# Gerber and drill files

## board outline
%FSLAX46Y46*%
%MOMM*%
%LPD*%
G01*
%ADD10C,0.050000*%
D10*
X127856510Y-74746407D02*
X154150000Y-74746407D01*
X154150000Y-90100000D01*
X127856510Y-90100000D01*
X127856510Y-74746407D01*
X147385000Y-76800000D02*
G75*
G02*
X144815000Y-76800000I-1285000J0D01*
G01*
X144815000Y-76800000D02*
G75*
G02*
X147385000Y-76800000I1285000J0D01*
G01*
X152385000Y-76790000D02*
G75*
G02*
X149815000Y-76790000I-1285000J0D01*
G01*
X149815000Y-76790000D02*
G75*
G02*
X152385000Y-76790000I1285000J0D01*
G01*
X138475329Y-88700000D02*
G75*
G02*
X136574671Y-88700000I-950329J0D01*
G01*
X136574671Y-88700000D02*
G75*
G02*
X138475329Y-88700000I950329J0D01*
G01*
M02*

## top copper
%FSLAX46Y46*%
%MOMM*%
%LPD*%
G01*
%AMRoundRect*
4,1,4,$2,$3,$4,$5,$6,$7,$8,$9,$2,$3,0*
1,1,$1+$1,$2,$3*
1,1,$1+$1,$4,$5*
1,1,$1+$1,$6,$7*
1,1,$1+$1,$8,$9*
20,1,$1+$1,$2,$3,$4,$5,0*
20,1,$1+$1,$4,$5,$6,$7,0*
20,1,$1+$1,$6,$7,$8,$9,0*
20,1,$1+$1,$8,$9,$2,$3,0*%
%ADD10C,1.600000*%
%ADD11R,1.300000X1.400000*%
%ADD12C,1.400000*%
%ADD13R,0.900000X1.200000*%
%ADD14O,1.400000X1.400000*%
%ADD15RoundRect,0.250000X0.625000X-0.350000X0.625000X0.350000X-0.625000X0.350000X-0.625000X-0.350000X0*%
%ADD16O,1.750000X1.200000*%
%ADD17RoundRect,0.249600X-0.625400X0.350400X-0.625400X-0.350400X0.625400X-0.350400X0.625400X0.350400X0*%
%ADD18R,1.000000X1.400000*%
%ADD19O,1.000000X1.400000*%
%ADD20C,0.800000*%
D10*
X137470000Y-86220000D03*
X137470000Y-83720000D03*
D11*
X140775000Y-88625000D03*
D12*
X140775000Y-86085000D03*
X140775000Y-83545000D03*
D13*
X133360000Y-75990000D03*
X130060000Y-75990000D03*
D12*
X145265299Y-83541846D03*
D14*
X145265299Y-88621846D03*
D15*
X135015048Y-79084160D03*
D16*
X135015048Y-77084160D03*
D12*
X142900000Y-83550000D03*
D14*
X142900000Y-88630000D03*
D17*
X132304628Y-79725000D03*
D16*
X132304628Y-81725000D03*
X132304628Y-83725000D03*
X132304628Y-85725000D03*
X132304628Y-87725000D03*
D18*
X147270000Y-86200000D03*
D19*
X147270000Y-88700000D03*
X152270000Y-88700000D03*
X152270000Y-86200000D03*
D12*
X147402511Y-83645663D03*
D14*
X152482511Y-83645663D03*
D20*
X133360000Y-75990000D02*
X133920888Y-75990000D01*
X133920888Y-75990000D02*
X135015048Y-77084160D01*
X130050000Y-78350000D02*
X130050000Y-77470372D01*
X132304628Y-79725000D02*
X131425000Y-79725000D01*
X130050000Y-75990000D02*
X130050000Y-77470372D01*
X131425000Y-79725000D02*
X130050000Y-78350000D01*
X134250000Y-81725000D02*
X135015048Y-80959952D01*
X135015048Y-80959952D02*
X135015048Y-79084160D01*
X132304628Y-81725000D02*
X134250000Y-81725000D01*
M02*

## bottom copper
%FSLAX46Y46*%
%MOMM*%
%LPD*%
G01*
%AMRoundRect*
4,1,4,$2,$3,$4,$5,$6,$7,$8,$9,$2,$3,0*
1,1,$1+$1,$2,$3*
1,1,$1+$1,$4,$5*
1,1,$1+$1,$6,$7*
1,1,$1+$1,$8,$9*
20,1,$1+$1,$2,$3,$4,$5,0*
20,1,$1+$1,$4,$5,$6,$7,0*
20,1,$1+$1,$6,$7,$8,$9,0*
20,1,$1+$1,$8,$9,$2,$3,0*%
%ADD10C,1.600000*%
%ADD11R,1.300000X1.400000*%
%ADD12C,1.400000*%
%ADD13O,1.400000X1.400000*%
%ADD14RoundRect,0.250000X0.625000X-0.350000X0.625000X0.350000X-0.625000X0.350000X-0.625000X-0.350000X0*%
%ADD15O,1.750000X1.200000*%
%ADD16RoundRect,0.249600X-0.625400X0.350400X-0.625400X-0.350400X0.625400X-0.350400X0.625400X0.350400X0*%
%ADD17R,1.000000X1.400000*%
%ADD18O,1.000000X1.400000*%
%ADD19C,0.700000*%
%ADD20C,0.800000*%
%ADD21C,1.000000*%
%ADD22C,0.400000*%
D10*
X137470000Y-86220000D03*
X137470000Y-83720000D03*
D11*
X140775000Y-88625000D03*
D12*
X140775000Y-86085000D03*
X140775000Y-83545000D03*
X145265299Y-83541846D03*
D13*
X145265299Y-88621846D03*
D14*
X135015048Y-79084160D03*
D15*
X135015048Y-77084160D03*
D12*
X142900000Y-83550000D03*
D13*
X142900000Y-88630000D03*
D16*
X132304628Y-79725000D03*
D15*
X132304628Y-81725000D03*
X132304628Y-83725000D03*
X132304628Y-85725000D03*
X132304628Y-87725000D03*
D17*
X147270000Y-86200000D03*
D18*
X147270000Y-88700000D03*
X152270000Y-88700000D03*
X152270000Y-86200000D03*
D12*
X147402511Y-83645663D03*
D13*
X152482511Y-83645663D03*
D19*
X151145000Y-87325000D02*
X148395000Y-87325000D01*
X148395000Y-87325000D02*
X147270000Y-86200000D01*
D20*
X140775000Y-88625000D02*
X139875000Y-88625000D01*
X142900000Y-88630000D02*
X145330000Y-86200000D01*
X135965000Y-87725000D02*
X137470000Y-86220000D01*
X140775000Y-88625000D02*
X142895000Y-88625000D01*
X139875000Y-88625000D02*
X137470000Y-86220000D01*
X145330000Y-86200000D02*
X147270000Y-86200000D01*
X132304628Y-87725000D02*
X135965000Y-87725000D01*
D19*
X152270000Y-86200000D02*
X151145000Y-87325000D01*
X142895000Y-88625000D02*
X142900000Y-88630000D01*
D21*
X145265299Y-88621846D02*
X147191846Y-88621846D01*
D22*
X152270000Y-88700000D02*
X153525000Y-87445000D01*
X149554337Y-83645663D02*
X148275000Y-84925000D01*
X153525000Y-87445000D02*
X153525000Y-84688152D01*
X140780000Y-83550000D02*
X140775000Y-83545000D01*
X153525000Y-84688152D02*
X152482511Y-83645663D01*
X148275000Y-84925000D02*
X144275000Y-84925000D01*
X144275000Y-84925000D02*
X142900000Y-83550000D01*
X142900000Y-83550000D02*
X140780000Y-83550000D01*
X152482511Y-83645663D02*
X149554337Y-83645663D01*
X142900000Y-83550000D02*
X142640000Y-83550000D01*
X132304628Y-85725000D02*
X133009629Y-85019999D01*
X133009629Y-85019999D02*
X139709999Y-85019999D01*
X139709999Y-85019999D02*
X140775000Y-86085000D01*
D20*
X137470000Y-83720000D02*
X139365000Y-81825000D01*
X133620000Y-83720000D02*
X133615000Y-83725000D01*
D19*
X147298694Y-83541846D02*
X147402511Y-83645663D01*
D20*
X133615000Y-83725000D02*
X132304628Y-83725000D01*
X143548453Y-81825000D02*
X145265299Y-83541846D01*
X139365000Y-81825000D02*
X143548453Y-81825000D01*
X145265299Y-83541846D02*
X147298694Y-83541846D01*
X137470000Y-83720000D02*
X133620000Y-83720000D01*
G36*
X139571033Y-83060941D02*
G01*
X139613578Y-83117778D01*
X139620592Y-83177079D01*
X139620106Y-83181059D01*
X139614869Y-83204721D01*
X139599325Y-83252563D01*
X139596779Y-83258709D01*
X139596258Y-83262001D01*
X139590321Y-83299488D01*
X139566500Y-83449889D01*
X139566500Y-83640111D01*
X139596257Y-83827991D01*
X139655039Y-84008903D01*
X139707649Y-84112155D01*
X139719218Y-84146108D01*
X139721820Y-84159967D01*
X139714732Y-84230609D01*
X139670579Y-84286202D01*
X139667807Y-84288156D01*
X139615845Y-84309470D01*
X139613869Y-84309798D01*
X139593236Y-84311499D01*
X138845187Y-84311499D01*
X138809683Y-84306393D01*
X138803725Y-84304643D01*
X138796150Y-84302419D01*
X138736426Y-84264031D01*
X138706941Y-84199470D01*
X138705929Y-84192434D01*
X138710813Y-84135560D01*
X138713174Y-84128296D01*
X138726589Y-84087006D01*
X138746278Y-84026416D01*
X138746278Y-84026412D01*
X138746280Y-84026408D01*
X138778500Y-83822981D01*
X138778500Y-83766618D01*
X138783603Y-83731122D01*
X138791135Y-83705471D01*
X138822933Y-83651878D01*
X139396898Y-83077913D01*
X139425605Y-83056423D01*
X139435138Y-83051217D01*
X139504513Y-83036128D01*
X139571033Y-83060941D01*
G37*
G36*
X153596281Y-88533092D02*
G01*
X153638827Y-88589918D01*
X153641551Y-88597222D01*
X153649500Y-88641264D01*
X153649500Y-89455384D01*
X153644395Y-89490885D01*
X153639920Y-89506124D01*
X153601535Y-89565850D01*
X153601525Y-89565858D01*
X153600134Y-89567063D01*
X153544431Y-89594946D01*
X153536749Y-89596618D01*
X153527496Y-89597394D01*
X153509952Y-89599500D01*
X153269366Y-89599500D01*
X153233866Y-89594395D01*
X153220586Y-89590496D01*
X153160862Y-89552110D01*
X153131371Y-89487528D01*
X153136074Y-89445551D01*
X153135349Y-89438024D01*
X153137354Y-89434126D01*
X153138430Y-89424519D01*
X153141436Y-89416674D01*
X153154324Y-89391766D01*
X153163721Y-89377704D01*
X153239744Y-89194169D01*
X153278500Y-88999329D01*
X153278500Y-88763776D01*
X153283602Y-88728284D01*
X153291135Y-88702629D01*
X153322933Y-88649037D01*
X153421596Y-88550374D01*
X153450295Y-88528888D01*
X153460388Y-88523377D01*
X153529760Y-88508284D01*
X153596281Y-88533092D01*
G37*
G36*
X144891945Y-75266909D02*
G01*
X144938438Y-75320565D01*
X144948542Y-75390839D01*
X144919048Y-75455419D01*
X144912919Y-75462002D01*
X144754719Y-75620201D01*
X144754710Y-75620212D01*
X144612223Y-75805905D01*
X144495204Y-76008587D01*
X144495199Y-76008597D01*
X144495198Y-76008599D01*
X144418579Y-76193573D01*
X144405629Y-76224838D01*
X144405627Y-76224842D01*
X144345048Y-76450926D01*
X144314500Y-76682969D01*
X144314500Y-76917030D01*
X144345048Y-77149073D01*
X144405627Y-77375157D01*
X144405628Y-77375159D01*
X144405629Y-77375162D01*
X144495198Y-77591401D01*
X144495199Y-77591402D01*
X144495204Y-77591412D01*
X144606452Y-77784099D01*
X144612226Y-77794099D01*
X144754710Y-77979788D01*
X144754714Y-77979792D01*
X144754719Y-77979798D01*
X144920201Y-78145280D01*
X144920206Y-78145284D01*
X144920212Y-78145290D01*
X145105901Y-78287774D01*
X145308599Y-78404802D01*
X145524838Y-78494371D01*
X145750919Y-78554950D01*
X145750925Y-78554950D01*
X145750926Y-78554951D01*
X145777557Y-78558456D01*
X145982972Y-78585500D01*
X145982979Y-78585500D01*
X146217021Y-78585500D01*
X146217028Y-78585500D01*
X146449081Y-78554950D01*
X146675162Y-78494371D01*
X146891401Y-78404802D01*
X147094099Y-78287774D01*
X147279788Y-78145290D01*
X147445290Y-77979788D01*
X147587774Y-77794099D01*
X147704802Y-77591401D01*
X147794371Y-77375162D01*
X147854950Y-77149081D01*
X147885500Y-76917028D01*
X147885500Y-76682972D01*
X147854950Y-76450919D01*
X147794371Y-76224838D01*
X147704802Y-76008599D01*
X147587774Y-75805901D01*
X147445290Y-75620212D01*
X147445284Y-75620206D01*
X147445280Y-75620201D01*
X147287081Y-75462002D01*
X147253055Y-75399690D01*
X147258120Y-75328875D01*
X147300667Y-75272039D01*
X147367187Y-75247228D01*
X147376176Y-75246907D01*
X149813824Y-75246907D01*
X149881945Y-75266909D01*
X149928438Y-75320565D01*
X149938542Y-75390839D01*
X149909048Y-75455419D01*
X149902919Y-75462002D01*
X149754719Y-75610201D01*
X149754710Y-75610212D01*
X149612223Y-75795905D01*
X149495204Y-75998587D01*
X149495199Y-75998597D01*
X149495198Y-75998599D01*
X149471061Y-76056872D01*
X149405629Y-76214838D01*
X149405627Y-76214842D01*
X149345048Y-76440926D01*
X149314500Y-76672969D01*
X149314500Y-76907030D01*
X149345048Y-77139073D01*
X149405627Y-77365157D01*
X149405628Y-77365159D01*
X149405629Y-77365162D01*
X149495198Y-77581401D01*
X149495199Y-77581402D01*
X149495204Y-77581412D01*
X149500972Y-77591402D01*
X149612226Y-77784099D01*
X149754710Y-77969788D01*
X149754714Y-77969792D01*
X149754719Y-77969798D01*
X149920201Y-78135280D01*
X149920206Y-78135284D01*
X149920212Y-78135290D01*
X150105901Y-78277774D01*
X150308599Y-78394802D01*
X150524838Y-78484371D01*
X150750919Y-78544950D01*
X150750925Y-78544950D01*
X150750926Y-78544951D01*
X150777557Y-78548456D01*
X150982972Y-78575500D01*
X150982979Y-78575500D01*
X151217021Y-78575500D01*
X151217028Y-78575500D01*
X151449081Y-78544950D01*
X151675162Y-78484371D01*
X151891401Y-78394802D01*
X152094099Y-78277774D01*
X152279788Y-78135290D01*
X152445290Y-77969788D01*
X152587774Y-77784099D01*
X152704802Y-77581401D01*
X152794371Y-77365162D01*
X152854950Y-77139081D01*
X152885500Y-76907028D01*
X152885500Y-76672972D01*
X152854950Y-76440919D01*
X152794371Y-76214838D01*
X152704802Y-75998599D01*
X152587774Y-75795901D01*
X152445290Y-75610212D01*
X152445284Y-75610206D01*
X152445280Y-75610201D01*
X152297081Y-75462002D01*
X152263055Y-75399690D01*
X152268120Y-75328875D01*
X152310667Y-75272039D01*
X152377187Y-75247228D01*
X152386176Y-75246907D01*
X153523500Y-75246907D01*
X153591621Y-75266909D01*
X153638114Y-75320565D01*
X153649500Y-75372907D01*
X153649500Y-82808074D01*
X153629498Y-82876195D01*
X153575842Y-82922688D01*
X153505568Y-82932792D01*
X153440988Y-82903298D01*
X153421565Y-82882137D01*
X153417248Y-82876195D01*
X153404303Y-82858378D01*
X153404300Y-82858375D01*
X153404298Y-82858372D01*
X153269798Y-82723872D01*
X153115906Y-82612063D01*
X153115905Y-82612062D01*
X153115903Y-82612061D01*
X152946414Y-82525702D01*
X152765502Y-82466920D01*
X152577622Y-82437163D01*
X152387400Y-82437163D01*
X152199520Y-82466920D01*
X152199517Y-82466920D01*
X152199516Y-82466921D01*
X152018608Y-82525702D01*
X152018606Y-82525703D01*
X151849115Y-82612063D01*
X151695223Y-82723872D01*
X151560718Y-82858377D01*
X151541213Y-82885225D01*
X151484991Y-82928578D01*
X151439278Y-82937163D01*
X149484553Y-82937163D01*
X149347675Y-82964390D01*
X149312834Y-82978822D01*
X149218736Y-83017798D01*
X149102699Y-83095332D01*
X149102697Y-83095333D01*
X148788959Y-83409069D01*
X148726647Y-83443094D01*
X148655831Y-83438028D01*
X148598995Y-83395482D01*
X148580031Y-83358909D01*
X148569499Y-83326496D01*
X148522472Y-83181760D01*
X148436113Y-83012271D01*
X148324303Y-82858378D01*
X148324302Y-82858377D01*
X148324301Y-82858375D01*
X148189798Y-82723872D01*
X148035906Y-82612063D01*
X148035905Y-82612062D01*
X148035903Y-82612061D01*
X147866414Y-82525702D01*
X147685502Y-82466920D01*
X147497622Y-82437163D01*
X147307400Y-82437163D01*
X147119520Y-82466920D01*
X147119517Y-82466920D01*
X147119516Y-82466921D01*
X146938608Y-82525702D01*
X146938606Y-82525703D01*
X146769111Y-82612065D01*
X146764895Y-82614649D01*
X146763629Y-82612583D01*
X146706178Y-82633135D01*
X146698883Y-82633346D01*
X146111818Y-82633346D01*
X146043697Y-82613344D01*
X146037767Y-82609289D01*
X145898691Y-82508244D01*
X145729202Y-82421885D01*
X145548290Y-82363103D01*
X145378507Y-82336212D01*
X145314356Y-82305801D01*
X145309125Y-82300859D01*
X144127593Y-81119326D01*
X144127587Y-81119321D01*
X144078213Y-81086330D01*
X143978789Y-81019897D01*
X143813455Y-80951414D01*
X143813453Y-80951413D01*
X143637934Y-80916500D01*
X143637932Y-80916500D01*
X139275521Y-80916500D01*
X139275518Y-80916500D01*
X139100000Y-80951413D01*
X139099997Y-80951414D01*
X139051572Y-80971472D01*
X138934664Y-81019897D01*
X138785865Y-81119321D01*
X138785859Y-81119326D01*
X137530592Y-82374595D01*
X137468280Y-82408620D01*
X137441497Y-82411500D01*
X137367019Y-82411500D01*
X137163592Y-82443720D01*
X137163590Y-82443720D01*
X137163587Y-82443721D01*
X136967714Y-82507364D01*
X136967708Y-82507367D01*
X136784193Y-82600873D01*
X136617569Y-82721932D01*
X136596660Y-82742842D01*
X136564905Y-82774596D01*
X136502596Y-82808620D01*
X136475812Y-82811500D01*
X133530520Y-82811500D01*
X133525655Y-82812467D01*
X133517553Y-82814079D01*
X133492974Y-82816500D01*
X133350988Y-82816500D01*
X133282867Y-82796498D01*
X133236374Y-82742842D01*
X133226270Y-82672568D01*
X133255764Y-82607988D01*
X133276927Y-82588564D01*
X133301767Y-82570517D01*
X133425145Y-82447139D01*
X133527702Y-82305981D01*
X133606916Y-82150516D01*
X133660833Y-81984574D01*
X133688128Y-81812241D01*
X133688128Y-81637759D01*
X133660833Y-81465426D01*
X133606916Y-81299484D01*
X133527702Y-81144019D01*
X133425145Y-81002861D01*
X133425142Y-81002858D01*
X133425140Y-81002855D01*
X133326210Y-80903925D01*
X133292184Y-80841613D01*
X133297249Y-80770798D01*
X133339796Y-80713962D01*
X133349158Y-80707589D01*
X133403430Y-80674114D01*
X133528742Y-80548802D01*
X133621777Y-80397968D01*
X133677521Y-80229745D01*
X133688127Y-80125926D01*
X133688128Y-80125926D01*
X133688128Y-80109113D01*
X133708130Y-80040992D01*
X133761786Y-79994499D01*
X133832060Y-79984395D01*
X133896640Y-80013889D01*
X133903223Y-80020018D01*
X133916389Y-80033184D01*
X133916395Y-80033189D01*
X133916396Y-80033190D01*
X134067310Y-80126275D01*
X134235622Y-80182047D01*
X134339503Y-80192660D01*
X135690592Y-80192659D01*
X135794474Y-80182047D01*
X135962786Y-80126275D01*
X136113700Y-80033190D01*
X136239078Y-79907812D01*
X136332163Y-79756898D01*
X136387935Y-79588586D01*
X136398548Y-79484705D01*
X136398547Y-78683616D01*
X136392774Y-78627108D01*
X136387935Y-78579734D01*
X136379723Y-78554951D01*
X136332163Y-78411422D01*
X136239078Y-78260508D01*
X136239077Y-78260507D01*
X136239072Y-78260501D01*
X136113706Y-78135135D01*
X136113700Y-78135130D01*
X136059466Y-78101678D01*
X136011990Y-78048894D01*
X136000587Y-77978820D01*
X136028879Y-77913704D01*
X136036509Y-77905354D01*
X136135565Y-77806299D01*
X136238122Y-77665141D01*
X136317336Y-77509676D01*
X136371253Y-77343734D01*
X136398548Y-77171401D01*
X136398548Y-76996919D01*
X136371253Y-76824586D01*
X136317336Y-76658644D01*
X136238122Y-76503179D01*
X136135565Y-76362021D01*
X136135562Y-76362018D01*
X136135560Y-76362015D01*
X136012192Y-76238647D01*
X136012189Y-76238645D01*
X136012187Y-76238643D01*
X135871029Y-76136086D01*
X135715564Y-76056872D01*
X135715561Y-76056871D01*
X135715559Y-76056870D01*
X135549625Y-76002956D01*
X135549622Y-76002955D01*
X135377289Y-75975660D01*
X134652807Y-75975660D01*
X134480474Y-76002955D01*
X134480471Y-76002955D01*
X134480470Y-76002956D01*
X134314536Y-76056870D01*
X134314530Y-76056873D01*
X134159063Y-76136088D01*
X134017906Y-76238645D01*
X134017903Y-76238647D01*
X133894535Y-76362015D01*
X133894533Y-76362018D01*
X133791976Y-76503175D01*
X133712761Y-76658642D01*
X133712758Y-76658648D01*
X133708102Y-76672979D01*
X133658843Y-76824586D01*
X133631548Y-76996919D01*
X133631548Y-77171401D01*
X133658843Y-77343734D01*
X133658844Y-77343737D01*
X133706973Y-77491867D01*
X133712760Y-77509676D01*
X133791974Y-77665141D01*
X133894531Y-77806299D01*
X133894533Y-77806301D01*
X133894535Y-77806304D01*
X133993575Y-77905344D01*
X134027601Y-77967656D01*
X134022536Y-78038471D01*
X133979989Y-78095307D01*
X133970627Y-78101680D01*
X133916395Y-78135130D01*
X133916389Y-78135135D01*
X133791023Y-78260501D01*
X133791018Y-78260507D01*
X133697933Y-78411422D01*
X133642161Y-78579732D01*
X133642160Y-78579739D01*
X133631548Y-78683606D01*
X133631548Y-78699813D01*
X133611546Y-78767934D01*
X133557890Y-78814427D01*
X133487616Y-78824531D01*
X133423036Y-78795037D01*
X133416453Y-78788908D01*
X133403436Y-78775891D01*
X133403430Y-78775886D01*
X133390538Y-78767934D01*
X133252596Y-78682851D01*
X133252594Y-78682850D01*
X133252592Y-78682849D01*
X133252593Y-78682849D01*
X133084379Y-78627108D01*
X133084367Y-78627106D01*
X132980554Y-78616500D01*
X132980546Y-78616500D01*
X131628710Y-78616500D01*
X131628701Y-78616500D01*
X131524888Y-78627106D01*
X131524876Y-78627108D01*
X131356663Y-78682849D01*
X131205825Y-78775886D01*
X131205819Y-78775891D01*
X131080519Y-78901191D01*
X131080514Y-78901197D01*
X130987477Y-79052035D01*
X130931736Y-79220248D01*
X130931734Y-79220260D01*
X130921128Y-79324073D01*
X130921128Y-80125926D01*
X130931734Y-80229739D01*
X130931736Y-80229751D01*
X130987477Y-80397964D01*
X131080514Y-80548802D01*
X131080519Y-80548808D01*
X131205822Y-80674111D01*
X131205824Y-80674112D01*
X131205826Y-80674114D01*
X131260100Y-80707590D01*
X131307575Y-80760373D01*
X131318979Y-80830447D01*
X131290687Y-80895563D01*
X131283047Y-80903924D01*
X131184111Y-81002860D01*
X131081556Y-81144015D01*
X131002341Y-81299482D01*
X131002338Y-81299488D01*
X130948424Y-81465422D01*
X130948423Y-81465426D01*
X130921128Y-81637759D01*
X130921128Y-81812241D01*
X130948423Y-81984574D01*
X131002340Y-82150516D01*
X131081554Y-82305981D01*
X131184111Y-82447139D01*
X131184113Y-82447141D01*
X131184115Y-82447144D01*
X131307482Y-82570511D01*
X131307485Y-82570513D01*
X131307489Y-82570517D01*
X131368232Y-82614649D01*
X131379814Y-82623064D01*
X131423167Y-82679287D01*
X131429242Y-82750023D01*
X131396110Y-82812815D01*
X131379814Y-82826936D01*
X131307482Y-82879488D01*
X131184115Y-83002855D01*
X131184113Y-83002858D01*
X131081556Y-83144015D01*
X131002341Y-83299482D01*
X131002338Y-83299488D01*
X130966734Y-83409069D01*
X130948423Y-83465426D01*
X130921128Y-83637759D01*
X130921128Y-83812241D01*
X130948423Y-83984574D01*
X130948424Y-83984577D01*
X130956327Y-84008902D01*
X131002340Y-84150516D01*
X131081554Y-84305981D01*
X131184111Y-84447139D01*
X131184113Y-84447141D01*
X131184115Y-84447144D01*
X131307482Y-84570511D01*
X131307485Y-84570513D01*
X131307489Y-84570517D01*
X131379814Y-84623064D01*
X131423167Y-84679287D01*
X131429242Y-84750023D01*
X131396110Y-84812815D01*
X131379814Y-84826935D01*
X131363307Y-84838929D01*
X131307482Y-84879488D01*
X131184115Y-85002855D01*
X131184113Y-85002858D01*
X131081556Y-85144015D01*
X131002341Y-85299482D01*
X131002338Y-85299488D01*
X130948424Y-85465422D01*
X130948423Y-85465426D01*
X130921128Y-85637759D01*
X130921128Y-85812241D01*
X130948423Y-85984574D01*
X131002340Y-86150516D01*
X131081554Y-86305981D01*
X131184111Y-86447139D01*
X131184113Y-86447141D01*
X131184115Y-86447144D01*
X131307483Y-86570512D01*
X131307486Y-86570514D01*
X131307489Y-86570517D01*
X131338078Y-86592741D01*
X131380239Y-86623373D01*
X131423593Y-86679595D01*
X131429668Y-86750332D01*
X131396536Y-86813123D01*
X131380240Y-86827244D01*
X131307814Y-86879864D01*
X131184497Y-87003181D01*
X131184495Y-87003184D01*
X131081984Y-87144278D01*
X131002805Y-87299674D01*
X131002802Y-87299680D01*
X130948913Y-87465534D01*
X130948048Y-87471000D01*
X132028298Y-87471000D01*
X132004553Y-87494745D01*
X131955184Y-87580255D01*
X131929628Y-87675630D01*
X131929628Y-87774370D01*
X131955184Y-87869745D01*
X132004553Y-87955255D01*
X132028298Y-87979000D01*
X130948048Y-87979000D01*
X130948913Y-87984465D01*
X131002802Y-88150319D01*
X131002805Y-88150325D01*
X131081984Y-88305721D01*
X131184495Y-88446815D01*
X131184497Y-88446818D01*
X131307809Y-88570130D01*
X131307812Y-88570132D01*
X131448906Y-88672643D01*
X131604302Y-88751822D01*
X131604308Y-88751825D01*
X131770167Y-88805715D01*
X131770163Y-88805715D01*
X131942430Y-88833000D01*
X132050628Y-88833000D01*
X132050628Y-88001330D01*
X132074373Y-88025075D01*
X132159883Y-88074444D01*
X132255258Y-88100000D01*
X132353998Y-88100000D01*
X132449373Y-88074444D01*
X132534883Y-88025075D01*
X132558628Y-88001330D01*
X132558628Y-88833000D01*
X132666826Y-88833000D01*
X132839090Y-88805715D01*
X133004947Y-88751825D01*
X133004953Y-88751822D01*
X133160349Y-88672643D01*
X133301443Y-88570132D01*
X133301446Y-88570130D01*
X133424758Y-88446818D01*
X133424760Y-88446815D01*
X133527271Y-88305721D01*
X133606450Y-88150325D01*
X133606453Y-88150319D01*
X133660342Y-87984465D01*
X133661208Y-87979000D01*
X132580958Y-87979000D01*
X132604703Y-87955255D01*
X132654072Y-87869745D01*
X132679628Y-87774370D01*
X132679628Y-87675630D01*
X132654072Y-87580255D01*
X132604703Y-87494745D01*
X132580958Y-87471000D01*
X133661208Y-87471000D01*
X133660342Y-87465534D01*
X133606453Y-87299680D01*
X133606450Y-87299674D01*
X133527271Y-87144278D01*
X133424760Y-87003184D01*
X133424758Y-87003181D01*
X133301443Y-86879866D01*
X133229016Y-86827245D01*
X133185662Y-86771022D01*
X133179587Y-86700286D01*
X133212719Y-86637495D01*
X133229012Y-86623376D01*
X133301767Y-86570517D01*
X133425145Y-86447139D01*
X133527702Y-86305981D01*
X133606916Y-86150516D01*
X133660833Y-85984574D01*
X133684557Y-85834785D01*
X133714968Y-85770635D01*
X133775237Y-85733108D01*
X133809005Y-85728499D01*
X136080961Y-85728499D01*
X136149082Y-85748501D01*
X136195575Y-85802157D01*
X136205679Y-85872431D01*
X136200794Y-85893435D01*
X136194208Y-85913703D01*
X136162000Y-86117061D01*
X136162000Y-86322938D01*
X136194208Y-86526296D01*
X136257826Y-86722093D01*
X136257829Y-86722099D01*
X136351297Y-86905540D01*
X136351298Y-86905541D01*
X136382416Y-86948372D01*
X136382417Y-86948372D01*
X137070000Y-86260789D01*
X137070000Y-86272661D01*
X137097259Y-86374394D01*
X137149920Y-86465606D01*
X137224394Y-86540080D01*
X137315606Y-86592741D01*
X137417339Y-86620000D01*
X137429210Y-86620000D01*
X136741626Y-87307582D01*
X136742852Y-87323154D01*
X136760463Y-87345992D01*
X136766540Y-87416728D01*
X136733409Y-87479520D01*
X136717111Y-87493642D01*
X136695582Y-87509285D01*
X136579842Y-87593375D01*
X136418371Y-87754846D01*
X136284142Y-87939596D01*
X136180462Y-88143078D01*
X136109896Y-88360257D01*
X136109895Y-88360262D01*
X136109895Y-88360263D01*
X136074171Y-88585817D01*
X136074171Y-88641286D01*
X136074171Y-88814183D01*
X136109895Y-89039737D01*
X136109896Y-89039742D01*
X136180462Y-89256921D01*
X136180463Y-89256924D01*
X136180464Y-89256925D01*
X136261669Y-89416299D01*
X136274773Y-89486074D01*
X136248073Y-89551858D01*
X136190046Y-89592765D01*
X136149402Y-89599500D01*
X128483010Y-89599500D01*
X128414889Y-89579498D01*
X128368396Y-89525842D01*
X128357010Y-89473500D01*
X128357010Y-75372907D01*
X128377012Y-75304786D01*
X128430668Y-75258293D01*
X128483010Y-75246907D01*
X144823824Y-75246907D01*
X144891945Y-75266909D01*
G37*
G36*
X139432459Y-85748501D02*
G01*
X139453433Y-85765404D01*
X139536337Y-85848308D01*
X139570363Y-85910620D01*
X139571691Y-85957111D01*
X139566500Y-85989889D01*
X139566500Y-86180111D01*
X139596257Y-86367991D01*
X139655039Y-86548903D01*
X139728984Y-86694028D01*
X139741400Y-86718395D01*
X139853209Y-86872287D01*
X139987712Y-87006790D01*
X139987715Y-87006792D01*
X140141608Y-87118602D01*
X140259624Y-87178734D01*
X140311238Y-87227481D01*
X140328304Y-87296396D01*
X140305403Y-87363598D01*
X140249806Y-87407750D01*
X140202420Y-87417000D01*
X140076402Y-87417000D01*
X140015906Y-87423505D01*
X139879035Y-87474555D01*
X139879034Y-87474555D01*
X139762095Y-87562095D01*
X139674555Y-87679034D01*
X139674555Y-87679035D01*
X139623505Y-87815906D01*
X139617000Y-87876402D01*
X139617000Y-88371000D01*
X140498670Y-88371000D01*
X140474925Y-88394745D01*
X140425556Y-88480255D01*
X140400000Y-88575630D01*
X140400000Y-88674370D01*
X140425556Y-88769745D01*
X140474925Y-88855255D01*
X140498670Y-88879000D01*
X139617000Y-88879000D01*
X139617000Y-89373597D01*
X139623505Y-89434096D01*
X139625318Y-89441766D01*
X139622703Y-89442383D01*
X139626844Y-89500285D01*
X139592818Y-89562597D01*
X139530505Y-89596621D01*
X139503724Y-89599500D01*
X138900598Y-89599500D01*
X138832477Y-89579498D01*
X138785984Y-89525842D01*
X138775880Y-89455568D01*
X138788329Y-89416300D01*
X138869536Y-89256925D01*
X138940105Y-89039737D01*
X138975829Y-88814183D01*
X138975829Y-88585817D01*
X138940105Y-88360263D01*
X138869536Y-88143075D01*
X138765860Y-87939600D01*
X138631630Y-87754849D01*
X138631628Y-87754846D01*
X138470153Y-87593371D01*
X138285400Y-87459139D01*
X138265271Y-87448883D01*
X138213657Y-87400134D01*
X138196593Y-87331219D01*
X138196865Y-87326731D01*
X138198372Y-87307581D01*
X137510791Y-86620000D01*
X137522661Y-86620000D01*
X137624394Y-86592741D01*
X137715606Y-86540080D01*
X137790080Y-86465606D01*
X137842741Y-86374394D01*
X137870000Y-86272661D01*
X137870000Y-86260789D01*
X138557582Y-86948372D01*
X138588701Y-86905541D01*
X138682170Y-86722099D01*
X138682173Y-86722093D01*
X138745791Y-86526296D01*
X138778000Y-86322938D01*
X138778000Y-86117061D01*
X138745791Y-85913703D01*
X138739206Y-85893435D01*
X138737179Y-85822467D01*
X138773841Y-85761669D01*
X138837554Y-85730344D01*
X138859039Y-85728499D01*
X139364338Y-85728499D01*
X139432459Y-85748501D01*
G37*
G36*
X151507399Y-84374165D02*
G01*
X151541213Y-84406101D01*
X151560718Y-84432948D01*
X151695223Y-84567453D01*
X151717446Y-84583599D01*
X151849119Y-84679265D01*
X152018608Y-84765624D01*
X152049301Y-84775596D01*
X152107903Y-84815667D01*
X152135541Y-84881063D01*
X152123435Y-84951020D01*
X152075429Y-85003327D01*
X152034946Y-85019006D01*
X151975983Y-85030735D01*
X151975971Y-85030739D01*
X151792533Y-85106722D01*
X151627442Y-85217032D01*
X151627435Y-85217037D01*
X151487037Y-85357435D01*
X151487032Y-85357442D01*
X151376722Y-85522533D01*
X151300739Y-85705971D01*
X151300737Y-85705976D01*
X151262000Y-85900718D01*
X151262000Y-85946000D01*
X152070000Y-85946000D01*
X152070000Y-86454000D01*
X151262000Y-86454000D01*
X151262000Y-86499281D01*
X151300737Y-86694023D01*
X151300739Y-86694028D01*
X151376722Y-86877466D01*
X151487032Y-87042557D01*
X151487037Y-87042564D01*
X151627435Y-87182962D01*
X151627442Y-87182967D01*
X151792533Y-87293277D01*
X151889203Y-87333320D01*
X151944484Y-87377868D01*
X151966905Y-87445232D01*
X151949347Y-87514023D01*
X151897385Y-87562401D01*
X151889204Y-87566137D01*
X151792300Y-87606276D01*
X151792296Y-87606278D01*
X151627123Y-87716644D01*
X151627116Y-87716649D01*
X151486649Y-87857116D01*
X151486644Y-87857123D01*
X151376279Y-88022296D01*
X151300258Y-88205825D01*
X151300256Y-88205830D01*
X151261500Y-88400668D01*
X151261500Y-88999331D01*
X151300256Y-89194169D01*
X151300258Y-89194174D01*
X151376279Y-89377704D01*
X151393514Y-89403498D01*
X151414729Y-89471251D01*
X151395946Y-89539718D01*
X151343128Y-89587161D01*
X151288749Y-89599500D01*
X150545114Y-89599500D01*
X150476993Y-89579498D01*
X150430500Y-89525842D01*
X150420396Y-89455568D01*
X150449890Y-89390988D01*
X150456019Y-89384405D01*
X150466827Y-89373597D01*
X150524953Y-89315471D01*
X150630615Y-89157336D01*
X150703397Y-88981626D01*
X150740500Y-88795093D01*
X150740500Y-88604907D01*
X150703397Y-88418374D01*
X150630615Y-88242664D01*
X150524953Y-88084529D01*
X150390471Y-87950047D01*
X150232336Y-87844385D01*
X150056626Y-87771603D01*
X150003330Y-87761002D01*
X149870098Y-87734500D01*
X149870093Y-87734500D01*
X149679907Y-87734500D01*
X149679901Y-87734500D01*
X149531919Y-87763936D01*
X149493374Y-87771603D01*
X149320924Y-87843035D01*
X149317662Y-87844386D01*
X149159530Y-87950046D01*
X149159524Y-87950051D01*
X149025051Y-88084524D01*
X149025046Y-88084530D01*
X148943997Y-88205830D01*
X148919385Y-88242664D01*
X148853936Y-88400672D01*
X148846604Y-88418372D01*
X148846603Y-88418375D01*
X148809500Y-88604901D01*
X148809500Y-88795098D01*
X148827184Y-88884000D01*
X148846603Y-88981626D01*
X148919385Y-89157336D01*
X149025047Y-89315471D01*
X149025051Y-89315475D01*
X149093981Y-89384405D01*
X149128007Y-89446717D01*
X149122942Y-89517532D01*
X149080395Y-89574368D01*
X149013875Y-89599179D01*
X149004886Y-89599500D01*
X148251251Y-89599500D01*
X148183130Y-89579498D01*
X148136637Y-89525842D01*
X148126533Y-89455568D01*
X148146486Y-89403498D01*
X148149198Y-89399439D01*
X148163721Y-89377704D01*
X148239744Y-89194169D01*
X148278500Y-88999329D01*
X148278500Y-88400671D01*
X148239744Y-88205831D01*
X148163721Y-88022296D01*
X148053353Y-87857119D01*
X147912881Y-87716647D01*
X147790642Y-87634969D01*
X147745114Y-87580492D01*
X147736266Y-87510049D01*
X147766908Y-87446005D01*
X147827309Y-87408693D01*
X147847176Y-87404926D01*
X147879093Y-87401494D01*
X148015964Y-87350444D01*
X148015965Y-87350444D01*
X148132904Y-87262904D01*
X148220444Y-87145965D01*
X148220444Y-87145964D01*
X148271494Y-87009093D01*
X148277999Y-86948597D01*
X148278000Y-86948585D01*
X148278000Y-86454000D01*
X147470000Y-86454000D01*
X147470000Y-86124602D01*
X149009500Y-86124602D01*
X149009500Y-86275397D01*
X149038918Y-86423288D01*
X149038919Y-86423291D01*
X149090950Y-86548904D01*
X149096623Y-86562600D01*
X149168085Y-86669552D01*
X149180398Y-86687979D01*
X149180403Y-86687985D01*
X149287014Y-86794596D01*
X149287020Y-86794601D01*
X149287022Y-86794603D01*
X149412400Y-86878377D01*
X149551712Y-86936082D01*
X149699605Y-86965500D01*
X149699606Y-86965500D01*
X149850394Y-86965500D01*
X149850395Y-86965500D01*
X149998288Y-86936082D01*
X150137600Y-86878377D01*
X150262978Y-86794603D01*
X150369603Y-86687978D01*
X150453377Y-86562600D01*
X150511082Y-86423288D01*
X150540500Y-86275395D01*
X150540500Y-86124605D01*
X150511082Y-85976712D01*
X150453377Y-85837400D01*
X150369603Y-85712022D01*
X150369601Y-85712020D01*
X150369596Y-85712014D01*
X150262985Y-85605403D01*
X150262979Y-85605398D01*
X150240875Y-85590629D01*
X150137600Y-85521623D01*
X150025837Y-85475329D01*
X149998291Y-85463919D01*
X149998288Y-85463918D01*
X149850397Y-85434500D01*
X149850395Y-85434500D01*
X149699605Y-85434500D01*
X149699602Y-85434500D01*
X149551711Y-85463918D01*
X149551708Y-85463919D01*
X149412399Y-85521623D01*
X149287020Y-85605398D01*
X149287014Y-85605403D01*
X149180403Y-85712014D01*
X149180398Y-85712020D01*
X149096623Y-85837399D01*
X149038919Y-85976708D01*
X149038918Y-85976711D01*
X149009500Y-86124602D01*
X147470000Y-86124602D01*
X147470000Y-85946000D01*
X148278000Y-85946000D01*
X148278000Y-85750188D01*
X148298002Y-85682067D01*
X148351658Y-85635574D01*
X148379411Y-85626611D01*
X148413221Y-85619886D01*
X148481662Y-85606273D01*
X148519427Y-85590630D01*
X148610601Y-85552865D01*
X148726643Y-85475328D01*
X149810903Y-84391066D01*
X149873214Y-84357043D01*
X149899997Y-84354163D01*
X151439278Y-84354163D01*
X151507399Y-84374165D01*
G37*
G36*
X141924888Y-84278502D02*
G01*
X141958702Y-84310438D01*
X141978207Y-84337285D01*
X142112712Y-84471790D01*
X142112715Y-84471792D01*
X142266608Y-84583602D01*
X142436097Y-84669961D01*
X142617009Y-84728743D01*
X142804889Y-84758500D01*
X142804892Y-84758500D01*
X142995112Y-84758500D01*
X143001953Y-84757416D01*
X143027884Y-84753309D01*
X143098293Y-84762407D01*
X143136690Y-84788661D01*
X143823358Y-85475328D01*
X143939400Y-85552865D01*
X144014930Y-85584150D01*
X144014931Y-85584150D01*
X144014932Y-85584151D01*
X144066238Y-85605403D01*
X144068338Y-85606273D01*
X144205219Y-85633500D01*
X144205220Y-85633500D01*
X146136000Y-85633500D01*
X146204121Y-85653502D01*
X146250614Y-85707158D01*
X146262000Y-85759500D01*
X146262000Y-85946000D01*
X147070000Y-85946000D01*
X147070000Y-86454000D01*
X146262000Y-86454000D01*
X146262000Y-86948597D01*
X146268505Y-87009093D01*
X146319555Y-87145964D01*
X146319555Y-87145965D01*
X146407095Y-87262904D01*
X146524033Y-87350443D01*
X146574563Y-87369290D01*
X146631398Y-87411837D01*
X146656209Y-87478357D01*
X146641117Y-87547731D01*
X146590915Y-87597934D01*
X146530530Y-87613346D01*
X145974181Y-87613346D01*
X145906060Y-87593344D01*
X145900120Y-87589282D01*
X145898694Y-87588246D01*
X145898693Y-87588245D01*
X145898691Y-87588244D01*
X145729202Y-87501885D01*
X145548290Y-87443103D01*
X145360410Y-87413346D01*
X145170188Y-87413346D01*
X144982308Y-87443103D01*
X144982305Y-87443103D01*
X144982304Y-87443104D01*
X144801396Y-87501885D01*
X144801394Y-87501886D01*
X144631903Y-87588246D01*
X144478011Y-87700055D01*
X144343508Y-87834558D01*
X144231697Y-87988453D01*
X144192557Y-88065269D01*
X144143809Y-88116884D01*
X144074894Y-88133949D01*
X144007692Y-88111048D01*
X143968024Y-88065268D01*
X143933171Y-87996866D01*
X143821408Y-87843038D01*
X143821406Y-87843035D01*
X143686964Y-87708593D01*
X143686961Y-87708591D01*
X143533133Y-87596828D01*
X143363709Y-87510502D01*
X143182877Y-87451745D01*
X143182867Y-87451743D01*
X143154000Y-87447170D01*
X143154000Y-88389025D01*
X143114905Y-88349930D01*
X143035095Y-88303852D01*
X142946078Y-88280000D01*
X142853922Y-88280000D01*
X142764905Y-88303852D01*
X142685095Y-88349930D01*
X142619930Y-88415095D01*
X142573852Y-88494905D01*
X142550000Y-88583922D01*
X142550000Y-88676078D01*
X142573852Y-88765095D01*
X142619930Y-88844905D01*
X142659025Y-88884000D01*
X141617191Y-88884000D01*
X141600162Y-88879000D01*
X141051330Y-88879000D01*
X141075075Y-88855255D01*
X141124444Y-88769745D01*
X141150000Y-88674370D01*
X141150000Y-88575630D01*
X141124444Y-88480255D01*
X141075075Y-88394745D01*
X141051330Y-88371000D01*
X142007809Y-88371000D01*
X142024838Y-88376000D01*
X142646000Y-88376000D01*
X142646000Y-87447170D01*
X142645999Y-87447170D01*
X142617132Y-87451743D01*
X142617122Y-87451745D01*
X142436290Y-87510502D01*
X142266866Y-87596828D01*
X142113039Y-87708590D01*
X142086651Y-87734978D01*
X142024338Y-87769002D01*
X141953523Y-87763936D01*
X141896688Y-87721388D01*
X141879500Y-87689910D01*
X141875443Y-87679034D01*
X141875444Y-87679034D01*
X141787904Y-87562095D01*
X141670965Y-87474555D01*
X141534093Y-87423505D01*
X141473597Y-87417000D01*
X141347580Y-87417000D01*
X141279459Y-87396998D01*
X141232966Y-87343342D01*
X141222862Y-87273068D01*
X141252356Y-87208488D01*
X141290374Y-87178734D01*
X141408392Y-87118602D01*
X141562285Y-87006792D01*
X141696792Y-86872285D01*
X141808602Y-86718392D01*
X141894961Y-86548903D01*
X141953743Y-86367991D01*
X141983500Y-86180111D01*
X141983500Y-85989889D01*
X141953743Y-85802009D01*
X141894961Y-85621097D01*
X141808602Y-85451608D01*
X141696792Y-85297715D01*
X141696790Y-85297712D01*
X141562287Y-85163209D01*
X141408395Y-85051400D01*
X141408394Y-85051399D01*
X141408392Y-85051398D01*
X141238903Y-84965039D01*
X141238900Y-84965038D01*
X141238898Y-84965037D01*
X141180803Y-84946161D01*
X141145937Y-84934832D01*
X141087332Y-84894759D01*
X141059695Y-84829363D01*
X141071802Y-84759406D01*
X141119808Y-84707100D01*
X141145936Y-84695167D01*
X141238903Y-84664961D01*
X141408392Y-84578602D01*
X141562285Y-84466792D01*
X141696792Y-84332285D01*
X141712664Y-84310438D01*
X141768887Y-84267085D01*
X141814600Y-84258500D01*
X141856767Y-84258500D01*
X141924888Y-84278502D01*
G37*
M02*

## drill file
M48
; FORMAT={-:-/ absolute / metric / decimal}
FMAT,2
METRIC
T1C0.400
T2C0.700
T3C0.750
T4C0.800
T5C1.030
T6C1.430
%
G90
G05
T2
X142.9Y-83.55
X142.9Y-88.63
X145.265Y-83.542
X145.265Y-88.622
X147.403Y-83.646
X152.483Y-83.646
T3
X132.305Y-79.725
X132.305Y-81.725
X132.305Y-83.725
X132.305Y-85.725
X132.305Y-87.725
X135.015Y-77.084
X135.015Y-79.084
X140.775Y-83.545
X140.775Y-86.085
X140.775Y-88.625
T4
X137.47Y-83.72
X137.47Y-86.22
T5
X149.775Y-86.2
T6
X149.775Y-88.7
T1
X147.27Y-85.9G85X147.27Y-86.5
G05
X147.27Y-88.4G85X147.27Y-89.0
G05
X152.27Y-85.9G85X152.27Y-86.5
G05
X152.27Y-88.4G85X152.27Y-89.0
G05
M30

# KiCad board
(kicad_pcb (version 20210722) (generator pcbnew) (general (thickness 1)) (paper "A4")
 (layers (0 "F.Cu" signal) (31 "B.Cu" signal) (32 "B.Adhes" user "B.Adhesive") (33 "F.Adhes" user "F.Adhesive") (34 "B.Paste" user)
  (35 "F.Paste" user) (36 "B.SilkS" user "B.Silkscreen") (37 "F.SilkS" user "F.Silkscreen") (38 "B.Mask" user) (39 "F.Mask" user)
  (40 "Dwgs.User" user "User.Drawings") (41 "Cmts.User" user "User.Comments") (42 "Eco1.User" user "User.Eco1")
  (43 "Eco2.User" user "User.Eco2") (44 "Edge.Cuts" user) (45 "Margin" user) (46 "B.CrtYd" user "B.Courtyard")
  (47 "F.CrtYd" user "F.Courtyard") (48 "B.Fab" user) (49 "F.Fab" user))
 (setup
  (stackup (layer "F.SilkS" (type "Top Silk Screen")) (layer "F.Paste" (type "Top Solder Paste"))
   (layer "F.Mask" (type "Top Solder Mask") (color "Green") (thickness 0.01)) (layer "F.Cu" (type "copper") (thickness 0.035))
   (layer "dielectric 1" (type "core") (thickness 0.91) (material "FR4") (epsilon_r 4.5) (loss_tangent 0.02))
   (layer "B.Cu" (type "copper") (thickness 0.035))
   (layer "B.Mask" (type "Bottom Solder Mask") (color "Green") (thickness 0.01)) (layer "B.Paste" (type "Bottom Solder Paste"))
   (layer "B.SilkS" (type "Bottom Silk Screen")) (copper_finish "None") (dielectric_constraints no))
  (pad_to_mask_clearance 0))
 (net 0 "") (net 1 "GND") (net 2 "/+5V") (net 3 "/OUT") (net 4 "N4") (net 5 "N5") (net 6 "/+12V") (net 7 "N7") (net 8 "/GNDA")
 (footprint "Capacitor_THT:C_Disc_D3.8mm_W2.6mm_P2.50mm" (layer "F.Cu") (at 137.47 86.22 90)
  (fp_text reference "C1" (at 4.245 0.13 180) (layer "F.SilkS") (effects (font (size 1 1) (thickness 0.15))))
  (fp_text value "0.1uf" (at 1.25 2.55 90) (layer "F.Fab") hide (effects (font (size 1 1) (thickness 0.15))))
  (pad "1" thru_hole circle locked (at 0 0 90) (size 1.6 1.6) (drill 0.8) (layers *.Cu *.Mask) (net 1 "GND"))
  (pad "2" thru_hole circle locked (at 2.5 0 90) (size 1.6 1.6) (drill 0.8) (layers *.Cu *.Mask) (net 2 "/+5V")))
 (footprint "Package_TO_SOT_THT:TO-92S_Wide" (layer "F.Cu") (at 140.775 88.625 90)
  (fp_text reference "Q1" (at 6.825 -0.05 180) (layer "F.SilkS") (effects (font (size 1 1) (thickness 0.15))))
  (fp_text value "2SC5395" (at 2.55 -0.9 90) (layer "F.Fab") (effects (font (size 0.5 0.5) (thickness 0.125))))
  (pad "1" thru_hole rect locked (at 0 0 90) (size 1.4 1.3) (drill 0.75) (layers *.Cu *.Mask) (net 1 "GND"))
  (pad "2" thru_hole circle locked (at 2.54 0 90) (size 1.4 1.4) (drill 0.75) (layers *.Cu *.Mask) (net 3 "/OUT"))
  (pad "3" thru_hole circle locked (at 5.08 0 90) (size 1.4 1.4) (drill 0.75) (layers *.Cu *.Mask) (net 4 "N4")))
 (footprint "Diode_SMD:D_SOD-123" (layer "F.Cu") (at 131.71 75.99 180)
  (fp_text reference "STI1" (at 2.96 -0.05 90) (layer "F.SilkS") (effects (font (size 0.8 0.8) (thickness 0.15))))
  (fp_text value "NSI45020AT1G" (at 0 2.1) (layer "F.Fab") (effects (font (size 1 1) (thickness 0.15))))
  (pad "1" smd rect locked (at -1.65 0 180) (size 0.9 1.2) (layers "F.Cu" "F.Paste" "F.Mask") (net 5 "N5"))
  (pad "2" smd rect locked (at 1.65 0 180) (size 0.9 1.2) (layers "F.Cu" "F.Paste" "F.Mask") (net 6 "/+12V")))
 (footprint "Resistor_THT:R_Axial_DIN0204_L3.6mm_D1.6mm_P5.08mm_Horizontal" (layer "F.Cu") (at 145.265299 83.541846 -90)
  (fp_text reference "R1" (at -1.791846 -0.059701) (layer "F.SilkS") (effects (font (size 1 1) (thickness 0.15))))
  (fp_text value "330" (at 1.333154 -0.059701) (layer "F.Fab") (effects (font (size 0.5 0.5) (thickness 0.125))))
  (pad "1" thru_hole circle locked (at 0 0 270) (size 1.4 1.4) (drill 0.7) (layers *.Cu *.Mask) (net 2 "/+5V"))
  (pad "2" thru_hole oval locked (at 5.08 0 270) (size 1.4 1.4) (drill 0.7) (layers *.Cu *.Mask) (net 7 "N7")))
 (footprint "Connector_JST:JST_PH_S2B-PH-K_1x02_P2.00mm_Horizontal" (layer "F.Cu") (at 135.015048 79.08416 90)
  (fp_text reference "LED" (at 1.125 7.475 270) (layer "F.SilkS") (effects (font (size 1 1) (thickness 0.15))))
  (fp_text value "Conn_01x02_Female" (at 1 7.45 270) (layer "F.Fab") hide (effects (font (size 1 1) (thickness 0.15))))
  (pad "1" thru_hole roundrect locked (at 0 0 90) (size 1.2 1.75) (drill 0.75) (layers *.Cu *.Mask) (roundrect_rratio 0.2083333333)
   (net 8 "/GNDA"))
  (pad "2" thru_hole oval locked (at 2 0 90) (size 1.2 1.75) (drill 0.75) (layers *.Cu *.Mask) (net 5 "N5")))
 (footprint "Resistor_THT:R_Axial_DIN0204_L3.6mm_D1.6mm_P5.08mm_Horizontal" (layer "F.Cu") (at 142.9 83.55 -90)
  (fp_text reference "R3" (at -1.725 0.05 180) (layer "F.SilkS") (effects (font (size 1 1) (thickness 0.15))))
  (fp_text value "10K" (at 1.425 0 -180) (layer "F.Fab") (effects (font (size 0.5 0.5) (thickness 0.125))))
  (pad "1" thru_hole circle locked (at 0 0 270) (size 1.4 1.4) (drill 0.7) (layers *.Cu *.Mask) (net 4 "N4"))
  (pad "2" thru_hole oval locked (at 5.08 0 270) (size 1.4 1.4) (drill 0.7) (layers *.Cu *.Mask) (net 1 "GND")))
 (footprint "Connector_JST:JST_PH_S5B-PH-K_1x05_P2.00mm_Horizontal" (layer "F.Cu") (at 132.304628 79.725 -90)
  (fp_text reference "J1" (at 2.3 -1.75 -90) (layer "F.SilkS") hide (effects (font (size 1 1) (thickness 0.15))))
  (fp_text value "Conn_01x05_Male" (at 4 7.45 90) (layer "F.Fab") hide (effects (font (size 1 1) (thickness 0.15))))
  (pad "1" thru_hole roundrect locked (at 0 0 270) (size 1.2 1.75) (drill 0.75) (layers *.Cu *.Mask) (roundrect_rratio 0.208)
   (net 6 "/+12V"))
  (pad "2" thru_hole oval locked (at 2 0 270) (size 1.2 1.75) (drill 0.75) (layers *.Cu *.Mask) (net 8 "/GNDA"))
  (pad "3" thru_hole oval locked (at 4 0 270) (size 1.2 1.75) (drill 0.75) (layers *.Cu *.Mask) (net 2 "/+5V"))
  (pad "4" thru_hole oval locked (at 6 0 270) (size 1.2 1.75) (drill 0.75) (layers *.Cu *.Mask) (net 3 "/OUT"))
  (pad "5" thru_hole oval locked (at 8 0 270) (size 1.2 1.75) (drill 0.75) (layers *.Cu *.Mask) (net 1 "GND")))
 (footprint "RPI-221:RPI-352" (layer "F.Cu") (at 146.5 89.6)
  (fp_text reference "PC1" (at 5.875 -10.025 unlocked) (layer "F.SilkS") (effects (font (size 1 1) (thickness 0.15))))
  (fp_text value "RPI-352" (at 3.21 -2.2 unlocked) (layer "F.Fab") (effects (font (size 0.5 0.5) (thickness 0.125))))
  (pad "" np_thru_hole circle locked (at 3.275 -3.4) (size 1.03 1.03) (drill 1.03) (layers *.Mask))
  (pad "" np_thru_hole circle locked (at 3.275 -0.9) (size 1.43 1.43) (drill 1.43) (layers *.Mask))
  (pad "1" thru_hole rect locked (at 0.77 -3.4) (size 1 1.4) (drill oval 0.4 1) (layers *.Cu *.Mask) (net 1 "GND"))
  (pad "2" thru_hole oval locked (at 0.77 -0.9) (size 1 1.4) (drill oval 0.4 1) (layers *.Cu *.Mask) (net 7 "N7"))
  (pad "3" thru_hole oval locked (at 5.77 -0.9) (size 1 1.4) (drill oval 0.4 1) (layers *.Cu *.Mask) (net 4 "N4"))
  (pad "4" thru_hole oval locked (at 5.77 -3.4) (size 1 1.4) (drill oval 0.4 1) (layers *.Cu *.Mask) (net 1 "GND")))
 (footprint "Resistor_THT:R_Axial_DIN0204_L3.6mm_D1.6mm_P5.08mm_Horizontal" (layer "F.Cu") (at 147.402511 83.645663)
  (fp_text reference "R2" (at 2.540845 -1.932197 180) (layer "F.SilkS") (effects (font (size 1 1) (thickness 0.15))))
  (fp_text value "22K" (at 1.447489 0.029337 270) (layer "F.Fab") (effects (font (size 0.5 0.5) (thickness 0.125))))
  (pad "1" thru_hole circle locked (at 0 0) (size 1.4 1.4) (drill 0.7) (layers *.Cu *.Mask) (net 2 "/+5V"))
  (pad "2" thru_hole oval locked (at 5.08 0) (size 1.4 1.4) (drill 0.7) (layers *.Cu *.Mask) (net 4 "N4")))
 (gr_rect (start 127.85651 74.746407) (end 154.15 90.1) (layer "Edge.Cuts") (width 0.05) (fill none))
 (gr_circle (center 146.1 76.8) (end 147.385 76.8) (layer "Edge.Cuts") (width 0.05) (fill none))
 (gr_circle (center 151.1 76.79) (end 152.385 76.79) (layer "Edge.Cuts") (width 0.05) (fill none))
 (gr_circle (center 137.525 88.7) (end 138.475 88.675) (layer "Edge.Cuts") (width 0.05) (fill none))
 (segment (start 151.145 87.325) (end 148.395 87.325) (width 0.7) (layer "B.Cu") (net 1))
 (segment (start 148.395 87.325) (end 147.27 86.2) (width 0.7) (layer "B.Cu") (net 1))
 (segment (start 140.775 88.625) (end 139.875 88.625) (width 0.8) (layer "B.Cu") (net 1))
 (segment (start 142.9 88.63) (end 145.33 86.2) (width 0.8) (layer "B.Cu") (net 1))
 (segment (start 135.965 87.725) (end 137.47 86.22) (width 0.8) (layer "B.Cu") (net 1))
 (segment (start 140.775 88.625) (end 142.895 88.625) (width 0.8) (layer "B.Cu") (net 1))
 (segment (start 139.875 88.625) (end 137.47 86.22) (width 0.8) (layer "B.Cu") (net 1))
 (segment (start 145.33 86.2) (end 147.27 86.2) (width 0.8) (layer "B.Cu") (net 1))
 (segment (start 132.304628 87.725) (end 135.965 87.725) (width 0.8) (layer "B.Cu") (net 1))
 (segment (start 152.27 86.2) (end 151.145 87.325) (width 0.7) (layer "B.Cu") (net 1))
 (segment (start 142.895 88.625) (end 142.9 88.63) (width 0.7) (layer "B.Cu") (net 1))
 (segment (start 133.36 75.99) (end 133.920888 75.99) (width 0.8) (layer "F.Cu") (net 5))
 (segment (start 133.920888 75.99) (end 135.015048 77.08416) (width 0.8) (layer "F.Cu") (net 5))
 (segment (start 145.265299 88.621846) (end 147.191846 88.621846) (width 1) (layer "B.Cu") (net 7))
 (segment (start 152.27 88.7) (end 153.525 87.445) (width 0.4) (layer "B.Cu") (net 4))
 (segment (start 149.554337 83.645663) (end 148.275 84.925) (width 0.4) (layer "B.Cu") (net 4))
 (segment (start 153.525 87.445) (end 153.525 84.688152) (width 0.4) (layer "B.Cu") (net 4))
 (segment (start 140.78 83.55) (end 140.775 83.545) (width 0.4) (layer "B.Cu") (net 4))
 (segment (start 153.525 84.688152) (end 152.482511 83.645663) (width 0.4) (layer "B.Cu") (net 4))
 (segment (start 148.275 84.925) (end 144.275 84.925) (width 0.4) (layer "B.Cu") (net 4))
 (segment (start 144.275 84.925) (end 142.9 83.55) (width 0.4) (layer "B.Cu") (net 4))
 (segment (start 142.9 83.55) (end 140.78 83.55) (width 0.4) (layer "B.Cu") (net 4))
 (segment (start 152.482511 83.645663) (end 149.554337 83.645663) (width 0.4) (layer "B.Cu") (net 4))
 (segment (start 142.9 83.55) (end 142.64 83.55) (width 0.4) (layer "B.Cu") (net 4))
 (segment (start 132.304628 85.725) (end 133.009629 85.019999) (width 0.4) (layer "B.Cu") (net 3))
 (segment (start 133.009629 85.019999) (end 139.709999 85.019999) (width 0.4) (layer "B.Cu") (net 3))
 (segment (start 139.709999 85.019999) (end 140.775 86.085) (width 0.4) (layer "B.Cu") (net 3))
 (segment (start 130.05 78.35) (end 130.05 77.470372) (width 0.8) (layer "F.Cu") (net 6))
 (segment (start 132.304628 79.725) (end 131.425 79.725) (width 0.8) (layer "F.Cu") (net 6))
 (segment (start 130.05 75.99) (end 130.05 77.470372) (width 0.8) (layer "F.Cu") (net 6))
 (segment (start 131.425 79.725) (end 130.05 78.35) (width 0.8) (layer "F.Cu") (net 6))
 (segment (start 134.25 81.725) (end 135.015048 80.959952) (width 0.8) (layer "F.Cu") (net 8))
 (segment (start 135.015048 80.959952) (end 135.015048 79.08416) (width 0.8) (layer "F.Cu") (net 8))
 (segment (start 132.304628 81.725) (end 134.25 81.725) (width 0.8) (layer "F.Cu") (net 8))
 (segment (start 137.47 83.72) (end 139.365 81.825) (width 0.8) (layer "B.Cu") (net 2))
 (segment (start 133.62 83.72) (end 133.615 83.725) (width 0.8) (layer "B.Cu") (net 2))
 (segment (start 147.298694 83.541846) (end 147.402511 83.645663) (width 0.7) (layer "B.Cu") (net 2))
 (segment (start 133.615 83.725) (end 132.304628 83.725) (width 0.8) (layer "B.Cu") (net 2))
 (segment (start 143.548453 81.825) (end 145.265299 83.541846) (width 0.8) (layer "B.Cu") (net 2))
 (segment (start 139.365 81.825) (end 143.548453 81.825) (width 0.8) (layer "B.Cu") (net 2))
 (segment (start 145.265299 83.541846) (end 147.298694 83.541846) (width 0.8) (layer "B.Cu") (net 2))
 (segment (start 137.47 83.72) (end 133.62 83.72) (width 0.8) (layer "B.Cu") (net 2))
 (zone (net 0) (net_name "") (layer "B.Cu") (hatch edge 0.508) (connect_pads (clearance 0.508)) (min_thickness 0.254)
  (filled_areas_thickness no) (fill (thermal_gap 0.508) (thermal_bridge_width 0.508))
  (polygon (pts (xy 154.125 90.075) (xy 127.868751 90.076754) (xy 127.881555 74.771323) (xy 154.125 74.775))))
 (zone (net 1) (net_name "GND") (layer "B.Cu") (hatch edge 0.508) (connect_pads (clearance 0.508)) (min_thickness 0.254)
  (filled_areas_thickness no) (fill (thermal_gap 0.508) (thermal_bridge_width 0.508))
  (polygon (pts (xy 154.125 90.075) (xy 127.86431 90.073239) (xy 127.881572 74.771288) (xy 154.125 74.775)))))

